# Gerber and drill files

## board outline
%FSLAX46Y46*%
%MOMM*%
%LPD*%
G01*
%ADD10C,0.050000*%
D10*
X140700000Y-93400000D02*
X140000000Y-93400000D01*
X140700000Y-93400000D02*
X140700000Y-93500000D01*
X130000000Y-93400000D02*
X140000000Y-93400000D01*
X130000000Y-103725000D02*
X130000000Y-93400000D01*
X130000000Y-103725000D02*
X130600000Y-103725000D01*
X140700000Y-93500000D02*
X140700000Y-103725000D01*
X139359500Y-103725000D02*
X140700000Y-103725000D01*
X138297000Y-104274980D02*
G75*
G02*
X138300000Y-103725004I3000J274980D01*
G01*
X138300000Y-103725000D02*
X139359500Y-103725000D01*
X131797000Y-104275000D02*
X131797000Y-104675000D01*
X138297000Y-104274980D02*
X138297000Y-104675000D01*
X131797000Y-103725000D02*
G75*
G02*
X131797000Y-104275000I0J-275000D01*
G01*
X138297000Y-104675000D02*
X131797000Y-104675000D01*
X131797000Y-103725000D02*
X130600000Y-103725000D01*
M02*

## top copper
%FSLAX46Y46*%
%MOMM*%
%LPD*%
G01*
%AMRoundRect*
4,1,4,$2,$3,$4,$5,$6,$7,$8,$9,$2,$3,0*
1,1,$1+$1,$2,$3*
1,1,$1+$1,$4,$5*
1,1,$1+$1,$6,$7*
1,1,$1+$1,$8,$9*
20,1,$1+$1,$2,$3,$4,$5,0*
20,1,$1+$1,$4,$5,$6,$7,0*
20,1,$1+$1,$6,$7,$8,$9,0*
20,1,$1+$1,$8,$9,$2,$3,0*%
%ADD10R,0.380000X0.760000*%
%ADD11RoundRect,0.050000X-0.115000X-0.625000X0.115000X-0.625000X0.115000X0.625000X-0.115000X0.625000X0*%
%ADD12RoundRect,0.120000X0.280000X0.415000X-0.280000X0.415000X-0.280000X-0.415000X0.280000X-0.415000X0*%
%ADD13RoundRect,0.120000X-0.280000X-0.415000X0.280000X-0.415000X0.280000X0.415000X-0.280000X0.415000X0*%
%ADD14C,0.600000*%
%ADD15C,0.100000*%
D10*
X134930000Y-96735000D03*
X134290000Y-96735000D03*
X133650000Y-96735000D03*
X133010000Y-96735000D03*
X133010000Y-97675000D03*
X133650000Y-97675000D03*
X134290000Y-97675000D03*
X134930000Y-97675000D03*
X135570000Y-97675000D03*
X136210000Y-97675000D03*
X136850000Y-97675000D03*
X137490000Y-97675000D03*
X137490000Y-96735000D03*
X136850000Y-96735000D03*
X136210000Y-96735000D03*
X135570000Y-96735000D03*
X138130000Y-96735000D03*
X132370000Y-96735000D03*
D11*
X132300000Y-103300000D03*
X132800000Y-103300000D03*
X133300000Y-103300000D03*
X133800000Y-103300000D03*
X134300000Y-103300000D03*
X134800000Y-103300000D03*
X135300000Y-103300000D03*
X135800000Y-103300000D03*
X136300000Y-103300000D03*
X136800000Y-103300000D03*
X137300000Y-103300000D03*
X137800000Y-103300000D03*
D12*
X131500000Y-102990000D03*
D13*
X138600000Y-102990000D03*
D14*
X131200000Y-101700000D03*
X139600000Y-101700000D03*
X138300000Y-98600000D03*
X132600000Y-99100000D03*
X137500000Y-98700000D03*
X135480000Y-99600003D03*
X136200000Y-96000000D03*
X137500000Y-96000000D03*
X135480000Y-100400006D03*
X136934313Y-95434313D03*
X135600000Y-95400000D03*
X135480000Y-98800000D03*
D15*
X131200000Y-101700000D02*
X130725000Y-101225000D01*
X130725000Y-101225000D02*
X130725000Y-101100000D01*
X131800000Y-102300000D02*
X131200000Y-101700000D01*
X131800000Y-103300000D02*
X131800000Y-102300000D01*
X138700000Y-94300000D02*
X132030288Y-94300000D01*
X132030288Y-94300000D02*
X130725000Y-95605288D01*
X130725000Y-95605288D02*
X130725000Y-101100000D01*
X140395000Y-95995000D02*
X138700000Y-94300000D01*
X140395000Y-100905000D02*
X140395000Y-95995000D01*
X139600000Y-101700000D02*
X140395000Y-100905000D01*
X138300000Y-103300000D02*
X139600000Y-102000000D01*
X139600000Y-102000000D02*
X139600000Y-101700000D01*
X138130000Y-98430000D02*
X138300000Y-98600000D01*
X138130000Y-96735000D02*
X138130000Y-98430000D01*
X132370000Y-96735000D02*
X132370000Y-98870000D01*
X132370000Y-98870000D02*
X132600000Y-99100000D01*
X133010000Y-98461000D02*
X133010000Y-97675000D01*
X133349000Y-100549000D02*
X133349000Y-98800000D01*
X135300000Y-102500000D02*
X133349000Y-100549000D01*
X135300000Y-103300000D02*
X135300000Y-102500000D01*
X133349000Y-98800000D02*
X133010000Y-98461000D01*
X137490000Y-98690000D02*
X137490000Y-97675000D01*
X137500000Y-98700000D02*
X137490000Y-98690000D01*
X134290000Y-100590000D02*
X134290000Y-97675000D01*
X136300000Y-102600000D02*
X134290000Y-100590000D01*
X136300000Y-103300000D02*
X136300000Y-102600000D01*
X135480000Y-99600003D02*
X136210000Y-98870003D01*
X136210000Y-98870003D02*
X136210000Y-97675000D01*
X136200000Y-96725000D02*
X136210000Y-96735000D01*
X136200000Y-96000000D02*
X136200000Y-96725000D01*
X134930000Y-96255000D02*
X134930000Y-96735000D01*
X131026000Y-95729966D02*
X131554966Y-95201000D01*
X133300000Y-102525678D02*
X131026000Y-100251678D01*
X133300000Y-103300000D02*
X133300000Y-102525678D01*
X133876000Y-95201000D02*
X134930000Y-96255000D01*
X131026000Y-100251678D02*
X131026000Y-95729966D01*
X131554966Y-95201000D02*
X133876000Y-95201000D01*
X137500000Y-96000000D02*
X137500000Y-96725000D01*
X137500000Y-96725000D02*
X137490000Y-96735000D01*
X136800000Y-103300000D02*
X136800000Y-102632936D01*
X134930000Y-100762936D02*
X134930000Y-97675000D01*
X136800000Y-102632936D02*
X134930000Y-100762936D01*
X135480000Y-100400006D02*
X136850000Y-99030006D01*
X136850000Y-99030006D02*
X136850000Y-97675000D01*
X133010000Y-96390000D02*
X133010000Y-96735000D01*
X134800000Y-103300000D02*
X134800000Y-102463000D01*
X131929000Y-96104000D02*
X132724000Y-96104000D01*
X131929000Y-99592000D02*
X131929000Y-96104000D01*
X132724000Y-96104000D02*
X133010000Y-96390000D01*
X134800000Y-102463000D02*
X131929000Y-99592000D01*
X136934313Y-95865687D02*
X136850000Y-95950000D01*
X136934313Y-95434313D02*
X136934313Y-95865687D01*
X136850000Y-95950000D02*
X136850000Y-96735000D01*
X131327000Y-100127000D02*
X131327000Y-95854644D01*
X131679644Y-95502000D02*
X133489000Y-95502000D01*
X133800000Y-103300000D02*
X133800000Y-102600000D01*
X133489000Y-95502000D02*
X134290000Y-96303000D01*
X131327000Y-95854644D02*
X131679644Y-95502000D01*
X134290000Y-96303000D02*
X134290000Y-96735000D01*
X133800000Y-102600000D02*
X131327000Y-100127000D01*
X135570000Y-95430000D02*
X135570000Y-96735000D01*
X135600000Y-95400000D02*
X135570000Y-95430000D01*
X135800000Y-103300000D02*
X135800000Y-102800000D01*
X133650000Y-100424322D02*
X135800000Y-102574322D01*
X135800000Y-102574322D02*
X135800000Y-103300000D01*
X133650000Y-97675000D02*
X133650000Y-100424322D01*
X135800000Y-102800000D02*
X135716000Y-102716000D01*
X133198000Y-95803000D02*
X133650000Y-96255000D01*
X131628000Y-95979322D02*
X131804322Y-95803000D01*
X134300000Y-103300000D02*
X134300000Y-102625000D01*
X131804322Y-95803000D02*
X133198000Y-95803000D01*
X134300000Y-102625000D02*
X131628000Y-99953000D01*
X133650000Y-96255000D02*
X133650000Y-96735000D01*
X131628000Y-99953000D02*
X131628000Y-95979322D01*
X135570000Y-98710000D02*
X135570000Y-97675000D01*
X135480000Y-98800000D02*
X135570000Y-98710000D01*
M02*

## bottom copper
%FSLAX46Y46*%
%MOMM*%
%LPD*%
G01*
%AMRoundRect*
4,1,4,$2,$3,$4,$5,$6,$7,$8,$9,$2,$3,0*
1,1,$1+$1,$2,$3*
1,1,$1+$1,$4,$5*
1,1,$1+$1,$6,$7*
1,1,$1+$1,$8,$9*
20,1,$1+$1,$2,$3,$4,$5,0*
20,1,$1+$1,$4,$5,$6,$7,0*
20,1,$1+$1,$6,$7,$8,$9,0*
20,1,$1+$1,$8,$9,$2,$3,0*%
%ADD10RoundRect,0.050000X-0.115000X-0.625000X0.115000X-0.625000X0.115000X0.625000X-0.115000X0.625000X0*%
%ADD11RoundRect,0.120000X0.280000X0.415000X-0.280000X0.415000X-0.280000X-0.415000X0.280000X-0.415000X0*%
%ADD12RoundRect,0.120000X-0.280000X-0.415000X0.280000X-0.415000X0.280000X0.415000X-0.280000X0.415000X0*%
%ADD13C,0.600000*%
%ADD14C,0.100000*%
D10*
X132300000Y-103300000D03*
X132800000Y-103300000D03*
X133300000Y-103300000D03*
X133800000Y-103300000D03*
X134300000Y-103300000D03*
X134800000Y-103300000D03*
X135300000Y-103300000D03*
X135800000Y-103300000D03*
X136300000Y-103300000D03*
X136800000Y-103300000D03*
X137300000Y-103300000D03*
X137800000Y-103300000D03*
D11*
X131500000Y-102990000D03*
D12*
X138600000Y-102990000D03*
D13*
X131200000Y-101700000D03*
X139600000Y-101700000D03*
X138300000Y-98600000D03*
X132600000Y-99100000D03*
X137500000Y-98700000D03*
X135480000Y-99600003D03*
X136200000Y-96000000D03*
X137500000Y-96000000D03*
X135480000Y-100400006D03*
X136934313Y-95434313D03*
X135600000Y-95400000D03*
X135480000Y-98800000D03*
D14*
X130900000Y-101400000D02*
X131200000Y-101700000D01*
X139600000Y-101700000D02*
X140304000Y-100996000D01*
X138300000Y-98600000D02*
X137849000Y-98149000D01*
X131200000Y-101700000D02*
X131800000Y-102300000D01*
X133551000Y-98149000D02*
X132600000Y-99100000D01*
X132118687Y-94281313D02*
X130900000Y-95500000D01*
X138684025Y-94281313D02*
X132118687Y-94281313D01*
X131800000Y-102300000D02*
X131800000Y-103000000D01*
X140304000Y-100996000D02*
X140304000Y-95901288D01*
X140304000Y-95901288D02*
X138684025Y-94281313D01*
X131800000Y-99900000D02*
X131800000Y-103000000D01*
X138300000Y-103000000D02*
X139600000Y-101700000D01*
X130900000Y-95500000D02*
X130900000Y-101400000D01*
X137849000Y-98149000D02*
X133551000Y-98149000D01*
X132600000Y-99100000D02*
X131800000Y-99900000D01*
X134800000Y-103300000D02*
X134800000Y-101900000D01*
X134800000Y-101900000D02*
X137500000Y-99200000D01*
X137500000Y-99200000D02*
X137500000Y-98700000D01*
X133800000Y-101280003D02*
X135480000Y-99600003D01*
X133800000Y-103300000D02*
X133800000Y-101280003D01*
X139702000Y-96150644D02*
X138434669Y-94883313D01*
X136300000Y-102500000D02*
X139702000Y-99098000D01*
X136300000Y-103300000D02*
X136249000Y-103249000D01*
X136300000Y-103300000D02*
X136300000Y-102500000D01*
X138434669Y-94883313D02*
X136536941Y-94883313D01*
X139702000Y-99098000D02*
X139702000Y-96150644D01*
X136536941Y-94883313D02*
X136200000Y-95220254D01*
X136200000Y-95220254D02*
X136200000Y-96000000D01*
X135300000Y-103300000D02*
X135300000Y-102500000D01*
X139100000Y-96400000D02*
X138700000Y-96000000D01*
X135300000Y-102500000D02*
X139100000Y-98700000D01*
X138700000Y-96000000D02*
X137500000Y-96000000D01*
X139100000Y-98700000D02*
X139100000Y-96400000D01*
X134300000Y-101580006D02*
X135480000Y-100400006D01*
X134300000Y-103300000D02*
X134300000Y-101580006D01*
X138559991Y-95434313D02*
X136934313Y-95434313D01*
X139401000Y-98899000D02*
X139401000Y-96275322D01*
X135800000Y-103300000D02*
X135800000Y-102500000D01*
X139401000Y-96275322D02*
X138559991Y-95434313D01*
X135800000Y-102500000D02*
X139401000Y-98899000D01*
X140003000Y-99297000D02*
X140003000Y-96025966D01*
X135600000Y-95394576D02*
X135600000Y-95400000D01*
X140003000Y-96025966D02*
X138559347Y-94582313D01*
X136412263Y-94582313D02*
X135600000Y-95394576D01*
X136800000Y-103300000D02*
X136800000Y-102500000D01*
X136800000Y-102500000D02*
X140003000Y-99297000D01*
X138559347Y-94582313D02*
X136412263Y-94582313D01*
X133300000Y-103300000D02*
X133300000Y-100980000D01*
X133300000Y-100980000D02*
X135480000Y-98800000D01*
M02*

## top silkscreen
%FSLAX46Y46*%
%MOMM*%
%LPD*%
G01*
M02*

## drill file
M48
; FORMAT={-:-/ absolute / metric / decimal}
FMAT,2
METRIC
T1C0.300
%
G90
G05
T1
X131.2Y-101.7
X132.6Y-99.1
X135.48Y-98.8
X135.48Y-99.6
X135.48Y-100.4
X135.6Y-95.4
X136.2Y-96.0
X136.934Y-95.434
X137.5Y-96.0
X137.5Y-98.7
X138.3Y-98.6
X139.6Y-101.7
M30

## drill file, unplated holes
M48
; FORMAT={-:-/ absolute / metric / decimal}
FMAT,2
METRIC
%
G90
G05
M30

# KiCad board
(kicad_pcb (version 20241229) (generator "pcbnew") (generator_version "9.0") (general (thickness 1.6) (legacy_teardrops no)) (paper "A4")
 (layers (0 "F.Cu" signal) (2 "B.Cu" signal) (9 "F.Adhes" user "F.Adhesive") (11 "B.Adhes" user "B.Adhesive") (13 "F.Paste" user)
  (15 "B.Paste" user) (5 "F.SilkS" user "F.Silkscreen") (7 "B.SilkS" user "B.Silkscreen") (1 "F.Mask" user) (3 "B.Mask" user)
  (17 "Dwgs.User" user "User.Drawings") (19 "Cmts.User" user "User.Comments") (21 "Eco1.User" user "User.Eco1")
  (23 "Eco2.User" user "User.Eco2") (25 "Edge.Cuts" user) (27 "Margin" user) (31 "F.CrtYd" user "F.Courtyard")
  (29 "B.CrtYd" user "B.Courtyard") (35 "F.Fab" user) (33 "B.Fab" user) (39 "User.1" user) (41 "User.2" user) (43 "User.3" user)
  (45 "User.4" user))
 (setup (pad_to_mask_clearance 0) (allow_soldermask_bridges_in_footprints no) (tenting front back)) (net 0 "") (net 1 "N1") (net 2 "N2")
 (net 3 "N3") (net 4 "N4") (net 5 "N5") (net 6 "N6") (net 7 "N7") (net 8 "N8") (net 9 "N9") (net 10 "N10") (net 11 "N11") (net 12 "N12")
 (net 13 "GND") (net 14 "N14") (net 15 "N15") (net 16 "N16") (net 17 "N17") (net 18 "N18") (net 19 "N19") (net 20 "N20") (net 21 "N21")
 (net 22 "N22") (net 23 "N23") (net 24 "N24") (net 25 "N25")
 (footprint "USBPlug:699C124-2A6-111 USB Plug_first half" (layer "F.Cu") (at 134.8 100.3)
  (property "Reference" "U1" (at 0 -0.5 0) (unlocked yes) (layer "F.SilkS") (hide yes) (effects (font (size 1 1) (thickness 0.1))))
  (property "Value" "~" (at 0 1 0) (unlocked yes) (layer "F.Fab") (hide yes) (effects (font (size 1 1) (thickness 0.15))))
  (pad "0" smd roundrect (at -2.5 3) (size 0.33 1.35) (layers "F.Cu" "F.Mask" "F.Paste") (roundrect_rratio 0.1515151515) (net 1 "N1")
   (thermal_bridge_angle 45))
  (pad "1" smd roundrect (at -2 3) (size 0.33 1.35) (layers "F.Cu" "F.Mask" "F.Paste") (roundrect_rratio 0.1515151515) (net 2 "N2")
   (thermal_bridge_angle 45))
  (pad "2" smd roundrect (at -1.5 3) (size 0.33 1.35) (layers "F.Cu" "F.Mask" "F.Paste") (roundrect_rratio 0.1515151515) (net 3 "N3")
   (thermal_bridge_angle 45))
  (pad "3" smd roundrect (at -1 3) (size 0.33 1.35) (layers "F.Cu" "F.Mask" "F.Paste") (roundrect_rratio 0.1515151515) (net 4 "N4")
   (thermal_bridge_angle 45))
  (pad "4" smd roundrect (at -0.5 3) (size 0.33 1.35) (layers "F.Cu" "F.Mask" "F.Paste") (roundrect_rratio 0.1515151515) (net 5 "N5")
   (thermal_bridge_angle 45))
  (pad "5" smd roundrect (at 0 3) (size 0.33 1.35) (layers "F.Cu" "F.Mask" "F.Paste") (roundrect_rratio 0.1515151515) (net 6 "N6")
   (thermal_bridge_angle 45))
  (pad "6" smd roundrect (at 0.5 3) (size 0.33 1.35) (layers "F.Cu" "F.Mask" "F.Paste") (roundrect_rratio 0.1515151515) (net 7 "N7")
   (thermal_bridge_angle 45))
  (pad "7" smd roundrect (at 1 3) (size 0.33 1.35) (layers "F.Cu" "F.Mask" "F.Paste") (roundrect_rratio 0.1515151515) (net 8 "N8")
   (thermal_bridge_angle 45))
  (pad "8" smd roundrect (at 1.5 3) (size 0.33 1.35) (layers "F.Cu" "F.Mask" "F.Paste") (roundrect_rratio 0.1515151515) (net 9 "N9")
   (thermal_bridge_angle 45))
  (pad "9" smd roundrect (at 2 3) (size 0.33 1.35) (layers "F.Cu" "F.Mask" "F.Paste") (roundrect_rratio 0.1515151515) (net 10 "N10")
   (thermal_bridge_angle 45))
  (pad "10" smd roundrect (at 2.5 3) (size 0.33 1.35) (layers "F.Cu" "F.Mask" "F.Paste") (roundrect_rratio 0.1515151515) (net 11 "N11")
   (thermal_bridge_angle 45))
  (pad "11" smd roundrect (at 3 3) (size 0.33 1.35) (layers "F.Cu" "F.Mask" "F.Paste") (roundrect_rratio 0.1515151515) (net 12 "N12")
   (thermal_bridge_angle 45))
  (pad "24" smd roundrect (at -3 3 180) (size 0.8 1.07) (drill (offset 0.3 0.31)) (layers "F.Cu" "F.Mask" "F.Paste") (roundrect_rratio 0.15)
   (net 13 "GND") (thermal_bridge_angle 45))
  (pad "25" smd roundrect (at 3.5 3) (size 0.8 1.07) (drill (offset 0.3 -0.31)) (layers "F.Cu" "F.Mask" "F.Paste") (roundrect_rratio 0.15)
   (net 13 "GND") (thermal_bridge_angle 45)))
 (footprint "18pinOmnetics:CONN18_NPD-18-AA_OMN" (layer "F.Cu") (at 134.93 95.795 180)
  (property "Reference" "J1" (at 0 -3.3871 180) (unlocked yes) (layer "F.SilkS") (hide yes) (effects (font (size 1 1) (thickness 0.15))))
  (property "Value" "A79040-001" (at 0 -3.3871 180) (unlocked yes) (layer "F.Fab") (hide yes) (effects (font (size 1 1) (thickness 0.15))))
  (pad "0" smd rect (at 0 -0.94 180) (size 0.38 0.76) (layers "F.Cu" "F.Mask" "F.Paste") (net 3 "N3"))
  (pad "1" smd rect (at 0.64 -0.94 180) (size 0.38 0.76) (layers "F.Cu" "F.Mask" "F.Paste") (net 4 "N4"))
  (pad "2" smd rect (at 1.28 -0.94 180) (size 0.38 0.76) (layers "F.Cu" "F.Mask" "F.Paste") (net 5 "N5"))
  (pad "3" smd rect (at 1.92 -0.94 180) (size 0.38 0.76) (layers "F.Cu" "F.Mask" "F.Paste") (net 6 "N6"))
  (pad "4" smd rect (at 1.92 -1.88 180) (size 0.38 0.76) (layers "F.Cu" "F.Mask" "F.Paste") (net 7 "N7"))
  (pad "5" smd rect (at 1.28 -1.88 180) (size 0.38 0.76) (layers "F.Cu" "F.Mask" "F.Paste") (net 8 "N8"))
  (pad "6" smd rect (at 0.64 -1.88 180) (size 0.38 0.76) (layers "F.Cu" "F.Mask" "F.Paste") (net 9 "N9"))
  (pad "7" smd rect (at 0 -1.88 180) (size 0.38 0.76) (layers "F.Cu" "F.Mask" "F.Paste") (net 10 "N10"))
  (pad "8" smd rect (at -0.64 -1.88 180) (size 0.38 0.76) (layers "F.Cu" "F.Mask" "F.Paste") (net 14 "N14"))
  (pad "9" smd rect (at -1.28 -1.88 180) (size 0.38 0.76) (layers "F.Cu" "F.Mask" "F.Paste") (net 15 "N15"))
  (pad "10" smd rect (at -1.92 -1.88 180) (size 0.38 0.76) (layers "F.Cu" "F.Mask" "F.Paste") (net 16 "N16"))
  (pad "11" smd rect (at -2.56 -1.88 180) (size 0.38 0.76) (layers "F.Cu" "F.Mask" "F.Paste") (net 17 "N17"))
  (pad "12" smd rect (at -2.56 -0.94 180) (size 0.38 0.76) (layers "F.Cu" "F.Mask" "F.Paste") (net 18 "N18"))
  (pad "13" smd rect (at -1.92 -0.94 180) (size 0.38 0.76) (layers "F.Cu" "F.Mask" "F.Paste") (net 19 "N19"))
  (pad "14" smd rect (at -1.28 -0.94 180) (size 0.38 0.76) (layers "F.Cu" "F.Mask" "F.Paste") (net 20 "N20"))
  (pad "15" smd rect (at -0.64 -0.94 180) (size 0.38 0.76) (layers "F.Cu" "F.Mask" "F.Paste") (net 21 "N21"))
  (pad "16" smd rect (at -3.2 -0.94 180) (size 0.38 0.76) (layers "F.Cu" "F.Mask" "F.Paste") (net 13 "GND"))
  (pad "17" smd rect (at 2.56 -0.94 180) (size 0.38 0.76) (layers "F.Cu" "F.Mask" "F.Paste") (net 13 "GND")))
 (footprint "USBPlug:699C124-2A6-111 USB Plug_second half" (layer "B.Cu") (at 134.8 106.3)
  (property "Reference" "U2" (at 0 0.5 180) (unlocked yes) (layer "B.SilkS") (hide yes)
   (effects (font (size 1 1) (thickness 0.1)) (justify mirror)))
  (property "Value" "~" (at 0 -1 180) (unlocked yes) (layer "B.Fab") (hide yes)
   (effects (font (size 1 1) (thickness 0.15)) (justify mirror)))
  (pad "12" smd roundrect (at -2.5 -3) (size 0.33 1.35) (layers "B.Cu" "B.Mask" "B.Paste") (roundrect_rratio 0.1515151515) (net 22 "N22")
   (thermal_bridge_angle 45))
  (pad "13" smd roundrect (at -2 -3) (size 0.33 1.35) (layers "B.Cu" "B.Mask" "B.Paste") (roundrect_rratio 0.1515151515) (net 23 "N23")
   (thermal_bridge_angle 45))
  (pad "14" smd roundrect (at -1.5 -3) (size 0.33 1.35) (layers "B.Cu" "B.Mask" "B.Paste") (roundrect_rratio 0.1515151515) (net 14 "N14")
   (thermal_bridge_angle 45))
  (pad "15" smd roundrect (at -1 -3) (size 0.33 1.35) (layers "B.Cu" "B.Mask" "B.Paste") (roundrect_rratio 0.1515151515) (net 15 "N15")
   (thermal_bridge_angle 45))
  (pad "16" smd roundrect (at -0.5 -3) (size 0.33 1.35) (layers "B.Cu" "B.Mask" "B.Paste") (roundrect_rratio 0.1515151515) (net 16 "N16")
   (thermal_bridge_angle 45))
  (pad "17" smd roundrect (at 0 -3) (size 0.33 1.35) (layers "B.Cu" "B.Mask" "B.Paste") (roundrect_rratio 0.1515151515) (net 17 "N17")
   (thermal_bridge_angle 45))
  (pad "18" smd roundrect (at 0.5 -3) (size 0.33 1.35) (layers "B.Cu" "B.Mask" "B.Paste") (roundrect_rratio 0.1515151515) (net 18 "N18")
   (thermal_bridge_angle 45))
  (pad "19" smd roundrect (at 1 -3) (size 0.33 1.35) (layers "B.Cu" "B.Mask" "B.Paste") (roundrect_rratio 0.1515151515) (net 19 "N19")
   (thermal_bridge_angle 45))
  (pad "20" smd roundrect (at 1.5 -3) (size 0.33 1.35) (layers "B.Cu" "B.Mask" "B.Paste") (roundrect_rratio 0.1515151515) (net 20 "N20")
   (thermal_bridge_angle 45))
  (pad "21" smd roundrect (at 2 -3) (size 0.33 1.35) (layers "B.Cu" "B.Mask" "B.Paste") (roundrect_rratio 0.1515151515) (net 21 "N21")
   (thermal_bridge_angle 45))
  (pad "22" smd roundrect (at 2.5 -3) (size 0.33 1.35) (layers "B.Cu" "B.Mask" "B.Paste") (roundrect_rratio 0.1515151515) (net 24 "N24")
   (thermal_bridge_angle 45))
  (pad "23" smd roundrect (at 3 -3) (size 0.33 1.35) (layers "B.Cu" "B.Mask" "B.Paste") (roundrect_rratio 0.1515151515) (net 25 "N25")
   (thermal_bridge_angle 45))
  (pad "26" smd roundrect (at -3 -3.3 180) (size 0.8 1.07) (drill (offset 0.3 0.01)) (layers "B.Cu" "B.Mask" "B.Paste")
   (roundrect_rratio 0.15) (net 13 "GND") (thermal_bridge_angle 45))
  (pad "27" smd roundrect (at 3.5 -3.3) (size 0.8 1.07) (drill (offset 0.3 -0.01)) (layers "B.Cu" "B.Mask" "B.Paste")
   (roundrect_rratio 0.15) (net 13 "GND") (thermal_bridge_angle 45)))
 (gr_arc (start 138.297 104.27498) (mid 138.025 104) (end 138.3 103.725) (stroke (width 0.05) (type default)) (layer "Edge.Cuts"))
 (gr_line (start 130 103.725) (end 130 93.4) (stroke (width 0.05) (type default)) (layer "Edge.Cuts"))
 (gr_line (start 140.7 93.4) (end 140.7 93.5) (stroke (width 0.05) (type default)) (layer "Edge.Cuts"))
 (gr_line (start 140.7 93.4) (end 140 93.4) (stroke (width 0.05) (type default)) (layer "Edge.Cuts"))
 (gr_line (start 138.3 103.725) (end 139.3595 103.725) (stroke (width 0.05) (type default)) (layer "Edge.Cuts"))
 (gr_line (start 131.797 104.275) (end 131.797 104.675) (stroke (width 0.05) (type default)) (layer "Edge.Cuts"))
 (gr_line (start 130 103.725) (end 130.6 103.725) (stroke (width 0.05) (type default)) (layer "Edge.Cuts"))
 (gr_line (start 130 93.4) (end 140 93.4) (stroke (width 0.05) (type default)) (layer "Edge.Cuts"))
 (gr_line (start 138.297 104.27498) (end 138.297 104.675) (stroke (width 0.05) (type default)) (layer "Edge.Cuts"))
 (gr_arc (start 131.797 103.725) (mid 132.072 104) (end 131.797 104.275) (stroke (width 0.05) (type default)) (layer "Edge.Cuts"))
 (gr_line (start 140.7 93.5) (end 140.7 103.725) (stroke (width 0.05) (type default)) (layer "Edge.Cuts"))
 (gr_line (start 138.297 104.675) (end 131.797 104.675) (stroke (width 0.05) (type default)) (layer "Edge.Cuts"))
 (gr_line (start 131.797 103.725) (end 130.6 103.725) (stroke (width 0.05) (type default)) (layer "Edge.Cuts"))
 (gr_line (start 139.3595 103.725) (end 140.7 103.725) (stroke (width 0.05) (type default)) (layer "Edge.Cuts"))
 (segment (start 138.13 98.43) (end 138.3 98.6) (width 0.1) (layer "F.Cu") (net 13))
 (segment (start 139.6 101.7) (end 140.395 100.905) (width 0.1) (layer "F.Cu") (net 13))
 (segment (start 130.725 95.605288) (end 130.725 101.1) (width 0.1) (layer "F.Cu") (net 13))
 (segment (start 138.13 96.735) (end 138.13 98.43) (width 0.1) (layer "F.Cu") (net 13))
 (segment (start 132.37 96.735) (end 132.37 98.87) (width 0.1) (layer "F.Cu") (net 13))
 (segment (start 138.7 94.3) (end 132.030288 94.3) (width 0.1) (layer "F.Cu") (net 13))
 (segment (start 138.3 103.3) (end 139.6 102) (width 0.1) (layer "F.Cu") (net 13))
 (segment (start 132.030288 94.3) (end 130.725 95.605288) (width 0.1) (layer "F.Cu") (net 13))
 (segment (start 130.725 101.225) (end 130.725 101.1) (width 0.1) (layer "F.Cu") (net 13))
 (segment (start 139.6 102) (end 139.6 101.7) (width 0.1) (layer "F.Cu") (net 13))
 (segment (start 140.395 100.905) (end 140.395 95.995) (width 0.1) (layer "F.Cu") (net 13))
 (segment (start 131.8 103.3) (end 131.8 102.3) (width 0.1) (layer "F.Cu") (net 13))
 (segment (start 132.37 98.87) (end 132.6 99.1) (width 0.1) (layer "F.Cu") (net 13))
 (segment (start 131.8 102.3) (end 131.2 101.7) (width 0.1) (layer "F.Cu") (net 13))
 (segment (start 131.2 101.7) (end 130.725 101.225) (width 0.1) (layer "F.Cu") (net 13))
 (segment (start 140.395 95.995) (end 138.7 94.3) (width 0.1) (layer "F.Cu") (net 13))
 (via (at 131.2 101.7) (size 0.6) (drill 0.3) (layers "F.Cu" "B.Cu") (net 13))
 (via (at 138.3 98.6) (size 0.6) (drill 0.3) (layers "F.Cu" "B.Cu") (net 13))
 (via (at 139.6 101.7) (size 0.6) (drill 0.3) (layers "F.Cu" "B.Cu") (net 13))
 (via (at 132.6 99.1) (size 0.6) (drill 0.3) (layers "F.Cu" "B.Cu") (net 13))
 (segment (start 138.3 98.6) (end 137.849 98.149) (width 0.1) (layer "B.Cu") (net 13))
 (segment (start 131.2 101.7) (end 131.8 102.3) (width 0.1) (layer "B.Cu") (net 13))
 (segment (start 133.551 98.149) (end 132.6 99.1) (width 0.1) (layer "B.Cu") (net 13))
 (segment (start 132.118687 94.281313) (end 130.9 95.5) (width 0.1) (layer "B.Cu") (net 13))
 (segment (start 138.684025 94.281313) (end 132.118687 94.281313) (width 0.1) (layer "B.Cu") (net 13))
 (segment (start 131.8 102.3) (end 131.8 103) (width 0.1) (layer "B.Cu") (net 13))
 (segment (start 140.304 100.996) (end 140.304 95.901288) (width 0.1) (layer "B.Cu") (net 13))
 (segment (start 140.304 95.901288) (end 138.684025 94.281313) (width 0.1) (layer "B.Cu") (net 13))
 (segment (start 139.6 101.7) (end 140.304 100.996) (width 0.1) (layer "B.Cu") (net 13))
 (segment (start 130.9 101.4) (end 131.2 101.7) (width 0.1) (layer "B.Cu") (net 13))
 (segment (start 131.8 99.9) (end 131.8 103) (width 0.1) (layer "B.Cu") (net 13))
 (segment (start 138.3 103) (end 139.6 101.7) (width 0.1) (layer "B.Cu") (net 13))
 (segment (start 130.9 95.5) (end 130.9 101.4) (width 0.1) (layer "B.Cu") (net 13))
 (segment (start 137.849 98.149) (end 133.551 98.149) (width 0.1) (layer "B.Cu") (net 13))
 (segment (start 132.6 99.1) (end 131.8 99.9) (width 0.1) (layer "B.Cu") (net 13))
 (segment (start 133.01 98.461) (end 133.01 97.675) (width 0.1) (layer "F.Cu") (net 7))
 (segment (start 133.349 100.549) (end 133.349 98.8) (width 0.1) (layer "F.Cu") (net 7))
 (segment (start 135.3 102.5) (end 133.349 100.549) (width 0.1) (layer "F.Cu") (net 7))
 (segment (start 135.3 103.3) (end 135.3 102.5) (width 0.1) (layer "F.Cu") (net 7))
 (segment (start 133.349 98.8) (end 133.01 98.461) (width 0.1) (layer "F.Cu") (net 7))
 (segment (start 137.49 98.69) (end 137.49 97.675) (width 0.1) (layer "F.Cu") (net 17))
 (segment (start 137.5 98.7) (end 137.49 98.69) (width 0.1) (layer "F.Cu") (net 17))
 (via (at 137.5 98.7) (size 0.6) (drill 0.3) (layers "F.Cu" "B.Cu") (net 17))
 (segment (start 134.8 103.3) (end 134.8 101.9) (width 0.1) (layer "B.Cu") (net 17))
 (segment (start 134.8 101.9) (end 137.5 99.2) (width 0.1) (layer "B.Cu") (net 17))
 (segment (start 137.5 99.2) (end 137.5 98.7) (width 0.1) (layer "B.Cu") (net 17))
 (segment (start 134.29 100.59) (end 134.29 97.675) (width 0.1) (layer "F.Cu") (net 9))
 (segment (start 136.3 102.6) (end 134.29 100.59) (width 0.1) (layer "F.Cu") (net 9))
 (segment (start 136.3 103.3) (end 136.3 102.6) (width 0.1) (layer "F.Cu") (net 9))
 (segment (start 135.48 99.600003) (end 136.21 98.870003) (width 0.1) (layer "F.Cu") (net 15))
 (segment (start 136.21 98.870003) (end 136.21 97.675) (width 0.1) (layer "F.Cu") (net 15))
 (via (at 135.48 99.600003) (size 0.6) (drill 0.3) (layers "F.Cu" "B.Cu") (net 15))
 (segment (start 133.8 101.280003) (end 135.48 99.600003) (width 0.1) (layer "B.Cu") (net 15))
 (segment (start 133.8 103.3) (end 133.8 101.280003) (width 0.1) (layer "B.Cu") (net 15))
 (segment (start 136.2 96.725) (end 136.21 96.735) (width 0.1) (layer "F.Cu") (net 20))
 (segment (start 136.2 96) (end 136.2 96.725) (width 0.1) (layer "F.Cu") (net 20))
 (via (at 136.2 96) (size 0.6) (drill 0.3) (layers "F.Cu" "B.Cu") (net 20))
 (segment (start 139.702 96.150644) (end 138.434669 94.883313) (width 0.1) (layer "B.Cu") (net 20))
 (segment (start 136.3 102.5) (end 139.702 99.098) (width 0.1) (layer "B.Cu") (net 20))
 (segment (start 136.3 103.3) (end 136.249 103.249) (width 0.1) (layer "B.Cu") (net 20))
 (segment (start 136.3 103.3) (end 136.3 102.5) (width 0.1) (layer "B.Cu") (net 20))
 (segment (start 138.434669 94.883313) (end 136.536941 94.883313) (width 0.1) (layer "B.Cu") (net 20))
 (segment (start 139.702 99.098) (end 139.702 96.150644) (width 0.1) (layer "B.Cu") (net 20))
 (segment (start 136.536941 94.883313) (end 136.2 95.220254) (width 0.1) (layer "B.Cu") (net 20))
 (segment (start 136.2 95.220254) (end 136.2 96) (width 0.1) (layer "B.Cu") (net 20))
 (segment (start 134.93 96.255) (end 134.93 96.735) (width 0.1) (layer "F.Cu") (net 3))
 (segment (start 131.026 95.729966) (end 131.554966 95.201) (width 0.1) (layer "F.Cu") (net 3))
 (segment (start 133.3 102.525678) (end 131.026 100.251678) (width 0.1) (layer "F.Cu") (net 3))
 (segment (start 133.3 103.3) (end 133.3 102.525678) (width 0.1) (layer "F.Cu") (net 3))
 (segment (start 133.876 95.201) (end 134.93 96.255) (width 0.1) (layer "F.Cu") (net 3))
 (segment (start 131.026 100.251678) (end 131.026 95.729966) (width 0.1) (layer "F.Cu") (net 3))
 (segment (start 131.554966 95.201) (end 133.876 95.201) (width 0.1) (layer "F.Cu") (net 3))
 (segment (start 137.5 96) (end 137.5 96.725) (width 0.1) (layer "F.Cu") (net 18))
 (segment (start 137.5 96.725) (end 137.49 96.735) (width 0.1) (layer "F.Cu") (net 18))
 (via (at 137.5 96) (size 0.6) (drill 0.3) (layers "F.Cu" "B.Cu") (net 18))
 (segment (start 135.3 103.3) (end 135.3 102.5) (width 0.1) (layer "B.Cu") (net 18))
 (segment (start 139.1 96.4) (end 138.7 96) (width 0.1) (layer "B.Cu") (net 18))
 (segment (start 135.3 102.5) (end 139.1 98.7) (width 0.1) (layer "B.Cu") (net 18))
 (segment (start 138.7 96) (end 137.5 96) (width 0.1) (layer "B.Cu") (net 18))
 (segment (start 139.1 98.7) (end 139.1 96.4) (width 0.1) (layer "B.Cu") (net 18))
 (segment (start 136.8 103.3) (end 136.8 102.632936) (width 0.1) (layer "F.Cu") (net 10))
 (segment (start 134.93 100.762936) (end 134.93 97.675) (width 0.1) (layer "F.Cu") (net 10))
 (segment (start 136.8 102.632936) (end 134.93 100.762936) (width 0.1) (layer "F.Cu") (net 10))
 (segment (start 135.48 100.400006) (end 136.85 99.030006) (width 0.1) (layer "F.Cu") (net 16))
 (segment (start 136.85 99.030006) (end 136.85 97.675) (width 0.1) (layer "F.Cu") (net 16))
 (via (at 135.48 100.400006) (size 0.6) (drill 0.3) (layers "F.Cu" "B.Cu") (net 16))
 (segment (start 134.3 101.580006) (end 135.48 100.400006) (width 0.1) (layer "B.Cu") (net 16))
 (segment (start 134.3 103.3) (end 134.3 101.580006) (width 0.1) (layer "B.Cu") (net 16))
 (segment (start 133.01 96.39) (end 133.01 96.735) (width 0.1) (layer "F.Cu") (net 6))
 (segment (start 134.8 103.3) (end 134.8 102.463) (width 0.1) (layer "F.Cu") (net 6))
 (segment (start 131.929 96.104) (end 132.724 96.104) (width 0.1) (layer "F.Cu") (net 6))
 (segment (start 131.929 99.592) (end 131.929 96.104) (width 0.1) (layer "F.Cu") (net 6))
 (segment (start 132.724 96.104) (end 133.01 96.39) (width 0.1) (layer "F.Cu") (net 6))
 (segment (start 134.8 102.463) (end 131.929 99.592) (width 0.1) (layer "F.Cu") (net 6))
 (segment (start 136.934313 95.865687) (end 136.85 95.95) (width 0.1) (layer "F.Cu") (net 19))
 (segment (start 136.934313 95.434313) (end 136.934313 95.865687) (width 0.1) (layer "F.Cu") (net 19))
 (segment (start 136.85 95.95) (end 136.85 96.735) (width 0.1) (layer "F.Cu") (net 19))
 (via (at 136.934313 95.434313) (size 0.6) (drill 0.3) (layers "F.Cu" "B.Cu") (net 19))
 (segment (start 138.559991 95.434313) (end 136.934313 95.434313) (width 0.1) (layer "B.Cu") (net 19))
 (segment (start 139.401 98.899) (end 139.401 96.275322) (width 0.1) (layer "B.Cu") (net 19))
 (segment (start 135.8 103.3) (end 135.8 102.5) (width 0.1) (layer "B.Cu") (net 19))
 (segment (start 139.401 96.275322) (end 138.559991 95.434313) (width 0.1) (layer "B.Cu") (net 19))
 (segment (start 135.8 102.5) (end 139.401 98.899) (width 0.1) (layer "B.Cu") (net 19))
 (segment (start 131.327 100.127) (end 131.327 95.854644) (width 0.1) (layer "F.Cu") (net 4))
 (segment (start 131.679644 95.502) (end 133.489 95.502) (width 0.1) (layer "F.Cu") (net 4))
 (segment (start 133.8 103.3) (end 133.8 102.6) (width 0.1) (layer "F.Cu") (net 4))
 (segment (start 133.489 95.502) (end 134.29 96.303) (width 0.1) (layer "F.Cu") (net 4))
 (segment (start 131.327 95.854644) (end 131.679644 95.502) (width 0.1) (layer "F.Cu") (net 4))
 (segment (start 134.29 96.303) (end 134.29 96.735) (width 0.1) (layer "F.Cu") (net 4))
 (segment (start 133.8 102.6) (end 131.327 100.127) (width 0.1) (layer "F.Cu") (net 4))
 (segment (start 135.57 95.43) (end 135.57 96.735) (width 0.1) (layer "F.Cu") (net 21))
 (segment (start 135.6 95.4) (end 135.57 95.43) (width 0.1) (layer "F.Cu") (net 21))
 (via (at 135.6 95.4) (size 0.6) (drill 0.3) (layers "F.Cu" "B.Cu") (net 21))
 (segment (start 140.003 99.297) (end 140.003 96.025966) (width 0.1) (layer "B.Cu") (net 21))
 (segment (start 135.6 95.394576) (end 135.6 95.4) (width 0.1) (layer "B.Cu") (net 21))
 (segment (start 140.003 96.025966) (end 138.559347 94.582313) (width 0.1) (layer "B.Cu") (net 21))
 (segment (start 136.412263 94.582313) (end 135.6 95.394576) (width 0.1) (layer "B.Cu") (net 21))
 (segment (start 136.8 103.3) (end 136.8 102.5) (width 0.1) (layer "B.Cu") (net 21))
 (segment (start 136.8 102.5) (end 140.003 99.297) (width 0.1) (layer "B.Cu") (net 21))
 (segment (start 138.559347 94.582313) (end 136.412263 94.582313) (width 0.1) (layer "B.Cu") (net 21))
 (segment (start 135.8 103.3) (end 135.8 102.8) (width 0.1) (layer "F.Cu") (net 8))
 (segment (start 133.65 100.424322) (end 135.8 102.574322) (width 0.1) (layer "F.Cu") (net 8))
 (segment (start 135.8 102.574322) (end 135.8 103.3) (width 0.1) (layer "F.Cu") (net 8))
 (segment (start 133.65 97.675) (end 133.65 100.424322) (width 0.1) (layer "F.Cu") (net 8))
 (segment (start 135.8 102.8) (end 135.716 102.716) (width 0.1) (layer "F.Cu") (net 8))
 (segment (start 133.198 95.803) (end 133.65 96.255) (width 0.1) (layer "F.Cu") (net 5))
 (segment (start 131.628 95.979322) (end 131.804322 95.803) (width 0.1) (layer "F.Cu") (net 5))
 (segment (start 134.3 103.3) (end 134.3 102.625) (width 0.1) (layer "F.Cu") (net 5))
 (segment (start 131.804322 95.803) (end 133.198 95.803) (width 0.1) (layer "F.Cu") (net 5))
 (segment (start 134.3 102.625) (end 131.628 99.953) (width 0.1) (layer "F.Cu") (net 5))
 (segment (start 133.65 96.255) (end 133.65 96.735) (width 0.1) (layer "F.Cu") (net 5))
 (segment (start 131.628 99.953) (end 131.628 95.979322) (width 0.1) (layer "F.Cu") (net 5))
 (segment (start 135.57 98.71) (end 135.57 97.675) (width 0.1) (layer "F.Cu") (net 14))
 (segment (start 135.48 98.8) (end 135.57 98.71) (width 0.1) (layer "F.Cu") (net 14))
 (via (at 135.48 98.8) (size 0.6) (drill 0.3) (layers "F.Cu" "B.Cu") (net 14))
 (segment (start 133.3 103.3) (end 133.3 100.98) (width 0.1) (layer "B.Cu") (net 14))
 (segment (start 133.3 100.98) (end 135.48 98.8) (width 0.1) (layer "B.Cu") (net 14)))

